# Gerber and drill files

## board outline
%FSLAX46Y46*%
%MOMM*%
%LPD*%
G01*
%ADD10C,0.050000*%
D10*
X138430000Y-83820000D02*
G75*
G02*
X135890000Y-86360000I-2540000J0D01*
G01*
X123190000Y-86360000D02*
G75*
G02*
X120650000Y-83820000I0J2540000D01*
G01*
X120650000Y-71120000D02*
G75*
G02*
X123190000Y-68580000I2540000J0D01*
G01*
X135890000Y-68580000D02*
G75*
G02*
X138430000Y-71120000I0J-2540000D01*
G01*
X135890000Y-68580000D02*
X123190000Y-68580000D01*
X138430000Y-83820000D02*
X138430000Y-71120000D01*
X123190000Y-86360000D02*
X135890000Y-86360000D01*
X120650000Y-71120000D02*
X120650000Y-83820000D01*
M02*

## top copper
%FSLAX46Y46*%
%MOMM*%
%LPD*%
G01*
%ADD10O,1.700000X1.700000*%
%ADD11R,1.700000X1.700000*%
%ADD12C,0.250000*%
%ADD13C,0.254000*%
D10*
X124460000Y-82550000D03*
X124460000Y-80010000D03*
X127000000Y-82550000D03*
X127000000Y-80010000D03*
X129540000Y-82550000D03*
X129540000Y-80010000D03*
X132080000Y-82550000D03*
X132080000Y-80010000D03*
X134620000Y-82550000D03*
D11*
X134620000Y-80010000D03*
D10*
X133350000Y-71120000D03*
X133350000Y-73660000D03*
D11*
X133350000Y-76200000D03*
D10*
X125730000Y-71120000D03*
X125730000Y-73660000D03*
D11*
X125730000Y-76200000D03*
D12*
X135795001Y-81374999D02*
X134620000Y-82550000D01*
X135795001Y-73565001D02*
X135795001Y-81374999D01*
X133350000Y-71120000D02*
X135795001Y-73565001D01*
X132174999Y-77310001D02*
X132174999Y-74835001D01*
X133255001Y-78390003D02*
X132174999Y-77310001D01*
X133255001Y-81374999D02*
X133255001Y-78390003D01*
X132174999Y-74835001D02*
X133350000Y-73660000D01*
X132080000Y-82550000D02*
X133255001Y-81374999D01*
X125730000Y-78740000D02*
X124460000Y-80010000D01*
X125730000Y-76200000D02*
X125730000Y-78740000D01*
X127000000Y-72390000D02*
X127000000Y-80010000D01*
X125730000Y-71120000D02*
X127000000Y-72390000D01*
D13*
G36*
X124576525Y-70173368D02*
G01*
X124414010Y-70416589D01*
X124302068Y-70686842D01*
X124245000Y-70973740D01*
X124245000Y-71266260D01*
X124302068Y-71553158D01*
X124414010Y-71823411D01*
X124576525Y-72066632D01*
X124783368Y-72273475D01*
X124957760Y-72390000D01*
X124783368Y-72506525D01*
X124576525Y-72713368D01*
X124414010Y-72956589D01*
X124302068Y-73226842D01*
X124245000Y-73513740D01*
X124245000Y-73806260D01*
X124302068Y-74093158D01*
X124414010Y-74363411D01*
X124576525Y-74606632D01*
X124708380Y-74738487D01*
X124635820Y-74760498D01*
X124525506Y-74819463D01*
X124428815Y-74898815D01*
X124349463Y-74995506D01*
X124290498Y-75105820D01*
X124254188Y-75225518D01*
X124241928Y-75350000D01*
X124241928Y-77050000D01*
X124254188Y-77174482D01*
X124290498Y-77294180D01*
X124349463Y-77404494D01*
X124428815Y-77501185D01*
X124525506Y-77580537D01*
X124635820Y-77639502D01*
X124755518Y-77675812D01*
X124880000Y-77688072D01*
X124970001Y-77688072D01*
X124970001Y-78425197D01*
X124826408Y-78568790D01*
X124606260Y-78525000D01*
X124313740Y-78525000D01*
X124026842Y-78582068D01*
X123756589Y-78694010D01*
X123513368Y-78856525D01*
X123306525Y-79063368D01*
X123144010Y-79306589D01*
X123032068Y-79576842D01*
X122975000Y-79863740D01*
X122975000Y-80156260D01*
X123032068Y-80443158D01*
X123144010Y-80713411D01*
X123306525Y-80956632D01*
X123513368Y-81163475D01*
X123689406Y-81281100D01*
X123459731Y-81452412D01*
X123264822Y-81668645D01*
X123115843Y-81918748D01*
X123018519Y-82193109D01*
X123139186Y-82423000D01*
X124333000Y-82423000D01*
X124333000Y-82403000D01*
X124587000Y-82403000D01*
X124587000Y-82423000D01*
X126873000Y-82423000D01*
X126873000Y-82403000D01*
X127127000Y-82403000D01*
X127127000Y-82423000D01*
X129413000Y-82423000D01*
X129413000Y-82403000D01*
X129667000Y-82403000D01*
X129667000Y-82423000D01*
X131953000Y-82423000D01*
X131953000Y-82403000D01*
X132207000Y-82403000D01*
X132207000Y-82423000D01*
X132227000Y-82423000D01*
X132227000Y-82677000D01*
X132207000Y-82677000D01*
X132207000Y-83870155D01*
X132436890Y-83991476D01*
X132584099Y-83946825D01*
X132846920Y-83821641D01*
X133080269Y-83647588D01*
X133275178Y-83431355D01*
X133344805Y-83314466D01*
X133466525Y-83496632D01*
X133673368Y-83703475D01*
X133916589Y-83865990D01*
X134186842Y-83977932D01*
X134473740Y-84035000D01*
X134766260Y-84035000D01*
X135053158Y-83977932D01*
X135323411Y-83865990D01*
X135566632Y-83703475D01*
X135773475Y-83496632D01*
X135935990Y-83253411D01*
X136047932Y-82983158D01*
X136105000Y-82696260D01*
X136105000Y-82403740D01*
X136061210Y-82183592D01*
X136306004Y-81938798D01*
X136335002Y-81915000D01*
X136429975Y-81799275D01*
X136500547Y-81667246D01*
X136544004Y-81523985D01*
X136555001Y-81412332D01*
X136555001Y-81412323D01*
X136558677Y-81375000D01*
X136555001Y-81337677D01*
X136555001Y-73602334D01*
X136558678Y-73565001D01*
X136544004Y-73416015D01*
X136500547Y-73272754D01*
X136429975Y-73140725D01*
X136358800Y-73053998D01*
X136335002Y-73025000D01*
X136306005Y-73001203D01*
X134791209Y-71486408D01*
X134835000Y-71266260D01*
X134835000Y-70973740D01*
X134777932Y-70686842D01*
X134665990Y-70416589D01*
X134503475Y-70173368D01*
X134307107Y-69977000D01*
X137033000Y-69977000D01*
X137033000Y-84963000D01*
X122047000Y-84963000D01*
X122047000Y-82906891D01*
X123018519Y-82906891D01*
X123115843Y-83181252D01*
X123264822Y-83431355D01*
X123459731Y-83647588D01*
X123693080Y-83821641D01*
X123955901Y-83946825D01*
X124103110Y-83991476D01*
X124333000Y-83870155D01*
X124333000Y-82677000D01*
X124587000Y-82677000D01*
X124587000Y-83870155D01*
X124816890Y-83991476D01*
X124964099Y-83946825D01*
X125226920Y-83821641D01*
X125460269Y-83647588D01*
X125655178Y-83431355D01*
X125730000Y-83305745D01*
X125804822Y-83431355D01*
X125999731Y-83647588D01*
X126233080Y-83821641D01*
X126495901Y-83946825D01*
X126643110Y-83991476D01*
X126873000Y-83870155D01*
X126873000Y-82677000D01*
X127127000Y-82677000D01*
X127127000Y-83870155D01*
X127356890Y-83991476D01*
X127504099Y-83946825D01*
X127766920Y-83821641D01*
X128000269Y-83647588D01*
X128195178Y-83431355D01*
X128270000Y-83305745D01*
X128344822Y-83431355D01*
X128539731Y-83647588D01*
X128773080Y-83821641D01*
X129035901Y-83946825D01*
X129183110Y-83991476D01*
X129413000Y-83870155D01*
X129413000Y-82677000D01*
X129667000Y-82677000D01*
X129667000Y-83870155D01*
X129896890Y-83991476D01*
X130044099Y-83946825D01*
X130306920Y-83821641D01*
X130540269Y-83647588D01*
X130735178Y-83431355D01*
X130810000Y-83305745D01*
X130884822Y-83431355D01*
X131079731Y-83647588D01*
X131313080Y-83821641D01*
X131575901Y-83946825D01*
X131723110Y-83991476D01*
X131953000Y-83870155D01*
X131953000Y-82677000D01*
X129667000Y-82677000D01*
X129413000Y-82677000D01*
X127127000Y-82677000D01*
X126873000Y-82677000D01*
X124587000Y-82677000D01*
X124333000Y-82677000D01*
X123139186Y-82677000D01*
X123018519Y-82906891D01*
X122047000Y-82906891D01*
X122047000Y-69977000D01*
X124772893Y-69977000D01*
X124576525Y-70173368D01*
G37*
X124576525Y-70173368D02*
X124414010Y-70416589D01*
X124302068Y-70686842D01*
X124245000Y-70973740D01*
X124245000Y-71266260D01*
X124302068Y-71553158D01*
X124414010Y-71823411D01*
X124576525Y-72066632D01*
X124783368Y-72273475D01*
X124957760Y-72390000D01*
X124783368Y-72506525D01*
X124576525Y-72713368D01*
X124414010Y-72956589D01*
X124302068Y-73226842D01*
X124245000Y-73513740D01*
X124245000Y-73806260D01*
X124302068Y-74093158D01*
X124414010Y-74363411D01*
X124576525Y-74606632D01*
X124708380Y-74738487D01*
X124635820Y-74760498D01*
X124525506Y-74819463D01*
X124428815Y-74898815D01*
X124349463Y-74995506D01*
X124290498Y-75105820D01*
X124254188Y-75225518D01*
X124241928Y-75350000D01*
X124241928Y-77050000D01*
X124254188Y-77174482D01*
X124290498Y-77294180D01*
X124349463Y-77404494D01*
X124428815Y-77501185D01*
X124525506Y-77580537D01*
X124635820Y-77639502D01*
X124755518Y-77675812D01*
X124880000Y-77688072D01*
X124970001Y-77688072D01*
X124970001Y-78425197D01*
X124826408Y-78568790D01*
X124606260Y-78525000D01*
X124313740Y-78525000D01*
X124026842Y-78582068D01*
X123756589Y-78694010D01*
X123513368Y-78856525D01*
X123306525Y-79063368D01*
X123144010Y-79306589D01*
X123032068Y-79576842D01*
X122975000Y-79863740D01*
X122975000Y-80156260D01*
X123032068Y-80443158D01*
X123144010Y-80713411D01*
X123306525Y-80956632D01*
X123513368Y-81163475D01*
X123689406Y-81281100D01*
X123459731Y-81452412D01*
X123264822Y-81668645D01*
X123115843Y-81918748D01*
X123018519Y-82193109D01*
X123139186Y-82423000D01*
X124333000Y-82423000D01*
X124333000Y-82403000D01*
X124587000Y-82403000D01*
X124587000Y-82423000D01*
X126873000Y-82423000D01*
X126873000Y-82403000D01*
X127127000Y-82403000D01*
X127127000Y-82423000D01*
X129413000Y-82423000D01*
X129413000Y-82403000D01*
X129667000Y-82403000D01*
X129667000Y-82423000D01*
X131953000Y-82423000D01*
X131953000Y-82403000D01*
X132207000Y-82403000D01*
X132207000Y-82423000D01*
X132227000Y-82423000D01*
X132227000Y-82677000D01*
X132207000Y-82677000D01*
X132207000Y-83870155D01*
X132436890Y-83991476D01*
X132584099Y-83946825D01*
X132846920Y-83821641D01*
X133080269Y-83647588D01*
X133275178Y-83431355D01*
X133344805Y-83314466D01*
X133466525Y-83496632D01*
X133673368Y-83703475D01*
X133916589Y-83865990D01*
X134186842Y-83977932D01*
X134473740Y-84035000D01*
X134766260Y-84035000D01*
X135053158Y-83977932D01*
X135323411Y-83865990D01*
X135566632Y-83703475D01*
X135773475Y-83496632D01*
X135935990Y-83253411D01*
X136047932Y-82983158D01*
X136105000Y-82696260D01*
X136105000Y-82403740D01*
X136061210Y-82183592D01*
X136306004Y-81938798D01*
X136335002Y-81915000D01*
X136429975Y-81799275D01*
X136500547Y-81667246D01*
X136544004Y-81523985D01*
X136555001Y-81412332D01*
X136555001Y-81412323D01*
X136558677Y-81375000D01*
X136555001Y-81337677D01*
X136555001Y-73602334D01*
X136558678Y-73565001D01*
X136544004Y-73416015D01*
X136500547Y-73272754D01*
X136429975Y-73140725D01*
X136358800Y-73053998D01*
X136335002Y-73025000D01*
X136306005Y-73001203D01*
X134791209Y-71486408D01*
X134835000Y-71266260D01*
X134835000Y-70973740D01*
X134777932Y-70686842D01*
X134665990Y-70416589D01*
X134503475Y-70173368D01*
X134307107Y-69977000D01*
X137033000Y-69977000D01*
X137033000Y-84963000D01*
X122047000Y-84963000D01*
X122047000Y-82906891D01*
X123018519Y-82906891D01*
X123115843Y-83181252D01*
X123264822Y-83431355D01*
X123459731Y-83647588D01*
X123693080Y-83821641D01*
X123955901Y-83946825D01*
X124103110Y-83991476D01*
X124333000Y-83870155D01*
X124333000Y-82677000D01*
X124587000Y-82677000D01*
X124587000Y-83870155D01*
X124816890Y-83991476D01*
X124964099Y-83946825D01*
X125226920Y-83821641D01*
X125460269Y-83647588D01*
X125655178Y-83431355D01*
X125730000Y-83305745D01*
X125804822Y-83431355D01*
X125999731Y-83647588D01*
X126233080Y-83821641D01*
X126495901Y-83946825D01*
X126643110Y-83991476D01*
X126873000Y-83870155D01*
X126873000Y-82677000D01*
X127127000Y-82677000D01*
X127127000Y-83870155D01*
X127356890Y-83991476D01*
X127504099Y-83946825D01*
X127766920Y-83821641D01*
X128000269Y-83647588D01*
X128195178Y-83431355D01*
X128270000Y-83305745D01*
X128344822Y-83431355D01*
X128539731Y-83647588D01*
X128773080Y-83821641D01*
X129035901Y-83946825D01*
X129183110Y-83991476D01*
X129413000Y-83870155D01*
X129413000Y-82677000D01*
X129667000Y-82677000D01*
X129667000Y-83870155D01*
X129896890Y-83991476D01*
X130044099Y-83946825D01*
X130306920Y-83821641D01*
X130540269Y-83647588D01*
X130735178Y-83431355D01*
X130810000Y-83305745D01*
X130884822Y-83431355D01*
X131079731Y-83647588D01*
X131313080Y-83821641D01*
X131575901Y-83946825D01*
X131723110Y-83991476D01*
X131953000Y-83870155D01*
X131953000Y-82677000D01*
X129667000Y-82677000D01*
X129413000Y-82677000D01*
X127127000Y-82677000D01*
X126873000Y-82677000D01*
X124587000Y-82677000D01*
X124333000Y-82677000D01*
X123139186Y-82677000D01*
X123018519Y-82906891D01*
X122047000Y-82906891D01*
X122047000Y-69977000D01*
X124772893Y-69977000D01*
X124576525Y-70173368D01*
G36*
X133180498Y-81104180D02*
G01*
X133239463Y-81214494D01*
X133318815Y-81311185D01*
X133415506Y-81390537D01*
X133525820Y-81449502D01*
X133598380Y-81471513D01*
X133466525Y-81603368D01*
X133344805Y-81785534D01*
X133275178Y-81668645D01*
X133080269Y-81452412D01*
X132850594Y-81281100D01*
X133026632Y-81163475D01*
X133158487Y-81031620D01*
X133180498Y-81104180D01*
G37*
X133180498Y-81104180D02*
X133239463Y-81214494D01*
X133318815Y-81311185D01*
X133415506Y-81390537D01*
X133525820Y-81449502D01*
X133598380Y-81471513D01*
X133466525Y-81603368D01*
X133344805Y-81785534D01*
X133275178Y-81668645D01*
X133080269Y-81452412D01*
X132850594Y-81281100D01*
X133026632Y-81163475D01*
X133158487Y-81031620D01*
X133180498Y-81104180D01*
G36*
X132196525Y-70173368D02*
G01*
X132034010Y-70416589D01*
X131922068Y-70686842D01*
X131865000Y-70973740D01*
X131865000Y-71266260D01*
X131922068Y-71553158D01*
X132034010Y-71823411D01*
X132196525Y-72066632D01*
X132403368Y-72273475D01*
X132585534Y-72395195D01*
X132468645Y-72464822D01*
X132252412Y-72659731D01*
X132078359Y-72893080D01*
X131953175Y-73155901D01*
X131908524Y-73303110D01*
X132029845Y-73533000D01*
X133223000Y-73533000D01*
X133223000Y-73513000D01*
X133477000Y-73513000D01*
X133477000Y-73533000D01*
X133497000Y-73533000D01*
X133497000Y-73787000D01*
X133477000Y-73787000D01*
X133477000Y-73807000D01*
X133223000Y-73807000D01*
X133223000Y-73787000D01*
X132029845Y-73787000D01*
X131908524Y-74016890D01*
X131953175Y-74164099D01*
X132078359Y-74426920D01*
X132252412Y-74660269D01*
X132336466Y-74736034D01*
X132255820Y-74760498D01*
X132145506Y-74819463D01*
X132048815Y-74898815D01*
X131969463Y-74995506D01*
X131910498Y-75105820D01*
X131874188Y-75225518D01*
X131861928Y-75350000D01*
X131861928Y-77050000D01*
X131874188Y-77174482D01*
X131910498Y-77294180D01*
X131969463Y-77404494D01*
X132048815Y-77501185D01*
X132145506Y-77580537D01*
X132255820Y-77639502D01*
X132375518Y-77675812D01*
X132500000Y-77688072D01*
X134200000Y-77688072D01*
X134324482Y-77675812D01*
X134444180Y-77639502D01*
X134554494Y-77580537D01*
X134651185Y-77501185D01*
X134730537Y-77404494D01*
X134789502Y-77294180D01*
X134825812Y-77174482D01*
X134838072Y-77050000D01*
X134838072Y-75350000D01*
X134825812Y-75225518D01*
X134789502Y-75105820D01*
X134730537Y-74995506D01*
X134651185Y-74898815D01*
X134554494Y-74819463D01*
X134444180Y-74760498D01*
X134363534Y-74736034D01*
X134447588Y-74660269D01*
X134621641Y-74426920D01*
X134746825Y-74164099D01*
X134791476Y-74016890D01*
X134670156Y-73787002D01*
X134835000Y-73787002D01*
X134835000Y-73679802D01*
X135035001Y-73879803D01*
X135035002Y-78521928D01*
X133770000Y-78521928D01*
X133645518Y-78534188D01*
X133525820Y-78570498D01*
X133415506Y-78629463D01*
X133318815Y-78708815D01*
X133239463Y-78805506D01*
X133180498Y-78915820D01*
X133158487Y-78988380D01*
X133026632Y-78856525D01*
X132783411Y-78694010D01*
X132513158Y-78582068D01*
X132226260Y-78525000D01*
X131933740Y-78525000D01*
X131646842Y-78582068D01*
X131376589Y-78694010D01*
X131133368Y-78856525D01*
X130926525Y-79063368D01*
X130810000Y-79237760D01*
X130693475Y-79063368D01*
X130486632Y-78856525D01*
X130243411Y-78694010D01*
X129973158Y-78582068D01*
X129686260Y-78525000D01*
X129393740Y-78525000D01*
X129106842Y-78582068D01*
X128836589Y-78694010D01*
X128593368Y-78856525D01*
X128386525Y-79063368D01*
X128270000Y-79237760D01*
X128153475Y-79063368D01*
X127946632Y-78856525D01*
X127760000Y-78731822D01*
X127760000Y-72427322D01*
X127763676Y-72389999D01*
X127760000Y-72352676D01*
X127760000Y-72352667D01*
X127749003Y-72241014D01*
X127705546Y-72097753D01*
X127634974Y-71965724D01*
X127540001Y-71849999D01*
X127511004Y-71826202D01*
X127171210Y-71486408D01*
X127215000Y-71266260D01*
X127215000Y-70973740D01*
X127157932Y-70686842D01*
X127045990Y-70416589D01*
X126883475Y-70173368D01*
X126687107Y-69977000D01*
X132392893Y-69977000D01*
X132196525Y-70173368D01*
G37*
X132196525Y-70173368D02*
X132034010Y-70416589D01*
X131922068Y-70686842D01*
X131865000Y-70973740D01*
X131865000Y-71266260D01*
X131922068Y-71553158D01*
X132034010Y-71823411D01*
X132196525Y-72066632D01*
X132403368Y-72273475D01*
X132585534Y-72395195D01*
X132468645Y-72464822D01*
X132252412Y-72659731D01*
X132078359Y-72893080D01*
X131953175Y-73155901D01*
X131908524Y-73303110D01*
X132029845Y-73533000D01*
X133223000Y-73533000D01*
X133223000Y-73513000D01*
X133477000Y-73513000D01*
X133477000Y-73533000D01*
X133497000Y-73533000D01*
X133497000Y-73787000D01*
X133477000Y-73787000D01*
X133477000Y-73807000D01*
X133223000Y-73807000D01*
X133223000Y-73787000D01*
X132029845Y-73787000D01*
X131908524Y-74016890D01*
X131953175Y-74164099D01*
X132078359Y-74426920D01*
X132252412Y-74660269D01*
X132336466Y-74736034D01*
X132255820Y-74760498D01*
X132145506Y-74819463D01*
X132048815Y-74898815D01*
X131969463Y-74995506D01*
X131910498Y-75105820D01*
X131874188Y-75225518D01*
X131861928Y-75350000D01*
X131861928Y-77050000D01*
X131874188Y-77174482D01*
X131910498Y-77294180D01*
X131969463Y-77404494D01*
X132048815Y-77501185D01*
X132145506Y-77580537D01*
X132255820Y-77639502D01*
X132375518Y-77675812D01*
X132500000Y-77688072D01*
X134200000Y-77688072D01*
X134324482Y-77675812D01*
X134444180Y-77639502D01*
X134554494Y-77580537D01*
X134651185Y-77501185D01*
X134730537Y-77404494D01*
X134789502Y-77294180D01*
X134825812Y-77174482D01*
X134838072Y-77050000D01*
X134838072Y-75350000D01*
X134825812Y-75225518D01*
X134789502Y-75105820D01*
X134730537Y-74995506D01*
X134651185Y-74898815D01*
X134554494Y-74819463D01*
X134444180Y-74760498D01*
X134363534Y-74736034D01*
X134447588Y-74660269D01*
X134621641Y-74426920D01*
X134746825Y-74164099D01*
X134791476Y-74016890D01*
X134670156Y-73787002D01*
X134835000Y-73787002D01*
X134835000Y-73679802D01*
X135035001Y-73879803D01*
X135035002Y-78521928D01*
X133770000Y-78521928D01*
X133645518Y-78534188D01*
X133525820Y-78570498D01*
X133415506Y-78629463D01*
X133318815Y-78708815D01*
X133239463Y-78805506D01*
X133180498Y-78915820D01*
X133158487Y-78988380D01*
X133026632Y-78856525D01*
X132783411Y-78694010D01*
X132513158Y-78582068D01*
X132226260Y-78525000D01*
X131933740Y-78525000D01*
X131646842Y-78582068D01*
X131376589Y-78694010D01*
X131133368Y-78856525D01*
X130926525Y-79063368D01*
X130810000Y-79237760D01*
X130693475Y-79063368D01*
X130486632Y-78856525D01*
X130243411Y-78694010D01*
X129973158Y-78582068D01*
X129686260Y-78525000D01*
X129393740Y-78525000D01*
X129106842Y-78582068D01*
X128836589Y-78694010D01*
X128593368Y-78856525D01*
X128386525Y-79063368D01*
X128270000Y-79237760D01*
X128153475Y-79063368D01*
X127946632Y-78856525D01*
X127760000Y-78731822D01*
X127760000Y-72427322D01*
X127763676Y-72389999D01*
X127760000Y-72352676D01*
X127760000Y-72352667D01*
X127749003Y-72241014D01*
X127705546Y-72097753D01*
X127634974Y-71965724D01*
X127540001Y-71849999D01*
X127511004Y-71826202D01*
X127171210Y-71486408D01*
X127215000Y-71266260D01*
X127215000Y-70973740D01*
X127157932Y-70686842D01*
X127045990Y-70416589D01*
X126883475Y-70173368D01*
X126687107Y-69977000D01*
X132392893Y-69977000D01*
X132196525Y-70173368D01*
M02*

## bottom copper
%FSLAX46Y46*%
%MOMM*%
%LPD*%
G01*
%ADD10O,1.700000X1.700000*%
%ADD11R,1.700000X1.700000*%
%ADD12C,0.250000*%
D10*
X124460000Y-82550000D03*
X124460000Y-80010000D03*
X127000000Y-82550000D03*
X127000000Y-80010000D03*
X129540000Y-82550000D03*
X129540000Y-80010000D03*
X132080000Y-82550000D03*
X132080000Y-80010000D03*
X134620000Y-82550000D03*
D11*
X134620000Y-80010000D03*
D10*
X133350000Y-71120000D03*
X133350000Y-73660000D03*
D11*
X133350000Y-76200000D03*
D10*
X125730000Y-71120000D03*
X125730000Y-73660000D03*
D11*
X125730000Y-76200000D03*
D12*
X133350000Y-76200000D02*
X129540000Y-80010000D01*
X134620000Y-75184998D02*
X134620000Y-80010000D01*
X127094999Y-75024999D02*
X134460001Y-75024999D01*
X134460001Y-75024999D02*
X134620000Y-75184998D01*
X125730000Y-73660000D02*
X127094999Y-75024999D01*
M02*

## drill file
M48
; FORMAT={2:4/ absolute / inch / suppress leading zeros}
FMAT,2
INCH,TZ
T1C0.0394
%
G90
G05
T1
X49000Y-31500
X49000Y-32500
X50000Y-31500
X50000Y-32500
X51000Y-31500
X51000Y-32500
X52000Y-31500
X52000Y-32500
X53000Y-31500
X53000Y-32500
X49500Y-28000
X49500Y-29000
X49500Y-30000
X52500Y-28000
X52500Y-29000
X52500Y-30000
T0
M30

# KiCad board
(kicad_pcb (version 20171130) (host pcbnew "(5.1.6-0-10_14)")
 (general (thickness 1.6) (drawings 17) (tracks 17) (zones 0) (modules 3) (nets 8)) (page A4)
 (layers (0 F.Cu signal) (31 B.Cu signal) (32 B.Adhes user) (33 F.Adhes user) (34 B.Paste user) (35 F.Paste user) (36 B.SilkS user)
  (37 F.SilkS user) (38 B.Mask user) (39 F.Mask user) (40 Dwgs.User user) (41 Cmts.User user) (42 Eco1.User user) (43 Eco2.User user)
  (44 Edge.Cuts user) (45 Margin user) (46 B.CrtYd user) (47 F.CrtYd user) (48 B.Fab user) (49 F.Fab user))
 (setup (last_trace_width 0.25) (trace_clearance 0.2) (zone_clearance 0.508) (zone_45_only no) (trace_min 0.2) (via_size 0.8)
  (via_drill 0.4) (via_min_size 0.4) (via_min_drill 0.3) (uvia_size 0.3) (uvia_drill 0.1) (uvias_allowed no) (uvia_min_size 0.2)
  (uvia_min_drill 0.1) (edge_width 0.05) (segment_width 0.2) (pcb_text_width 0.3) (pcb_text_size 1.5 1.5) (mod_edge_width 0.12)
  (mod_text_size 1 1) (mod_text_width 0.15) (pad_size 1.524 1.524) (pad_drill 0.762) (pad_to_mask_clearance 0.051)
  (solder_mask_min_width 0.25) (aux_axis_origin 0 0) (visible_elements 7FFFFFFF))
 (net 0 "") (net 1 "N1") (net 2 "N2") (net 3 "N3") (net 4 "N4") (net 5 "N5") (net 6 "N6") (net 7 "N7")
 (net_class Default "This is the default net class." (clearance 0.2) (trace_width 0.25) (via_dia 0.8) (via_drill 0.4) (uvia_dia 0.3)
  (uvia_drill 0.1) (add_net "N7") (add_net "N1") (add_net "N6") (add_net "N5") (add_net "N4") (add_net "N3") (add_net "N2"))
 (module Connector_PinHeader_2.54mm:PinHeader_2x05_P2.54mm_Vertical (layer F.Cu) (at 134.62 80.01 270)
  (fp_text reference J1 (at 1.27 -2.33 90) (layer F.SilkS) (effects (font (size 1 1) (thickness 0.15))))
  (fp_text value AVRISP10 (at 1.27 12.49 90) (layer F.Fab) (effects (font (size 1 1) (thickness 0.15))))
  (pad 10 thru_hole oval (at 2.54 10.16 270) (size 1.7 1.7) (drill 1) (layers *.Cu *.Mask) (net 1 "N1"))
  (pad 9 thru_hole oval (at 0 10.16 270) (size 1.7 1.7) (drill 1) (layers *.Cu *.Mask) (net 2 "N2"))
  (pad 8 thru_hole oval (at 2.54 7.62 270) (size 1.7 1.7) (drill 1) (layers *.Cu *.Mask) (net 1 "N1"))
  (pad 7 thru_hole oval (at 0 7.62 270) (size 1.7 1.7) (drill 1) (layers *.Cu *.Mask) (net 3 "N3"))
  (pad 6 thru_hole oval (at 2.54 5.08 270) (size 1.7 1.7) (drill 1) (layers *.Cu *.Mask) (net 1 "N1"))
  (pad 5 thru_hole oval (at 0 5.08 270) (size 1.7 1.7) (drill 1) (layers *.Cu *.Mask) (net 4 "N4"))
  (pad 4 thru_hole oval (at 2.54 2.54 270) (size 1.7 1.7) (drill 1) (layers *.Cu *.Mask) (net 1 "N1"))
  (pad 3 thru_hole oval (at 0 2.54 270) (size 1.7 1.7) (drill 1) (layers *.Cu *.Mask) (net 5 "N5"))
  (pad 2 thru_hole oval (at 2.54 0 270) (size 1.7 1.7) (drill 1) (layers *.Cu *.Mask) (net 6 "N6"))
  (pad 1 thru_hole rect (at 0 0 270) (size 1.7 1.7) (drill 1) (layers *.Cu *.Mask) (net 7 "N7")))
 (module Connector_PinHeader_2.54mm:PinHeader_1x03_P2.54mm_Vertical (layer B.Cu) (at 133.35 76.2)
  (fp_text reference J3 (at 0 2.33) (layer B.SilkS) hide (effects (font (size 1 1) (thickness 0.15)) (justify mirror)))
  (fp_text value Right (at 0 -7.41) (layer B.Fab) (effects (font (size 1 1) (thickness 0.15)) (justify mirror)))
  (pad 3 thru_hole oval (at 0 -5.08) (size 1.7 1.7) (drill 1) (layers *.Cu *.Mask) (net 6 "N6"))
  (pad 2 thru_hole oval (at 0 -2.54) (size 1.7 1.7) (drill 1) (layers *.Cu *.Mask) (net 1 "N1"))
  (pad 1 thru_hole rect (at 0 0) (size 1.7 1.7) (drill 1) (layers *.Cu *.Mask) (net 4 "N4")))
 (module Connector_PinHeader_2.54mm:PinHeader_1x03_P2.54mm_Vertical (layer B.Cu) (at 125.73 76.2)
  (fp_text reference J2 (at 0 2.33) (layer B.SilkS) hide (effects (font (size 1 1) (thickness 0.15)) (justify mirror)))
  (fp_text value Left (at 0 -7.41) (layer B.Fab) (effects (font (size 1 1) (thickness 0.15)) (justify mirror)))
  (pad 3 thru_hole oval (at 0 -5.08) (size 1.7 1.7) (drill 1) (layers *.Cu *.Mask) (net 3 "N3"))
  (pad 2 thru_hole oval (at 0 -2.54) (size 1.7 1.7) (drill 1) (layers *.Cu *.Mask) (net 7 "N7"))
  (pad 1 thru_hole rect (at 0 0) (size 1.7 1.7) (drill 1) (layers *.Cu *.Mask) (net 2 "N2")))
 (gr_arc (start 135.89 83.82) (end 135.89 86.36) (angle -90) (layer Edge.Cuts) (width 0.05))
 (gr_arc (start 123.19 83.82) (end 120.65 83.82) (angle -90) (layer Edge.Cuts) (width 0.05))
 (gr_arc (start 123.19 71.12) (end 123.19 68.58) (angle -90) (layer Edge.Cuts) (width 0.05))
 (gr_arc (start 135.89 71.12) (end 138.43 71.12) (angle -90) (layer Edge.Cuts) (width 0.05))
 (gr_line (start 135.89 68.58) (end 123.19 68.58) (layer Edge.Cuts) (width 0.05))
 (gr_line (start 138.43 83.82) (end 138.43 71.12) (layer Edge.Cuts) (width 0.05))
 (gr_line (start 123.19 86.36) (end 135.89 86.36) (layer Edge.Cuts) (width 0.05))
 (gr_line (start 120.65 71.12) (end 120.65 83.82) (layer Edge.Cuts) (width 0.05))
 (segment (start 133.35 76.2) (end 129.54 80.01) (width 0.25) (layer B.Cu) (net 4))
 (segment (start 135.795001 81.374999) (end 134.62 82.55) (width 0.25) (layer F.Cu) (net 6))
 (segment (start 135.795001 73.565001) (end 135.795001 81.374999) (width 0.25) (layer F.Cu) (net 6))
 (segment (start 133.35 71.12) (end 135.795001 73.565001) (width 0.25) (layer F.Cu) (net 6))
 (segment (start 134.62 75.184998) (end 134.62 80.01) (width 0.25) (layer B.Cu) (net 7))
 (segment (start 127.094999 75.024999) (end 134.460001 75.024999) (width 0.25) (layer B.Cu) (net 7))
 (segment (start 134.460001 75.024999) (end 134.62 75.184998) (width 0.25) (layer B.Cu) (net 7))
 (segment (start 125.73 73.66) (end 127.094999 75.024999) (width 0.25) (layer B.Cu) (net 7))
 (segment (start 132.174999 77.310001) (end 132.174999 74.835001) (width 0.25) (layer F.Cu) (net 1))
 (segment (start 133.255001 78.390003) (end 132.174999 77.310001) (width 0.25) (layer F.Cu) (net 1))
 (segment (start 133.255001 81.374999) (end 133.255001 78.390003) (width 0.25) (layer F.Cu) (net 1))
 (segment (start 132.174999 74.835001) (end 133.35 73.66) (width 0.25) (layer F.Cu) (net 1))
 (segment (start 132.08 82.55) (end 133.255001 81.374999) (width 0.25) (layer F.Cu) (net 1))
 (segment (start 125.73 78.74) (end 124.46 80.01) (width 0.25) (layer F.Cu) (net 2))
 (segment (start 125.73 76.2) (end 125.73 78.74) (width 0.25) (layer F.Cu) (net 2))
 (segment (start 127 72.39) (end 127 80.01) (width 0.25) (layer F.Cu) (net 3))
 (segment (start 125.73 71.12) (end 127 72.39) (width 0.25) (layer F.Cu) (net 3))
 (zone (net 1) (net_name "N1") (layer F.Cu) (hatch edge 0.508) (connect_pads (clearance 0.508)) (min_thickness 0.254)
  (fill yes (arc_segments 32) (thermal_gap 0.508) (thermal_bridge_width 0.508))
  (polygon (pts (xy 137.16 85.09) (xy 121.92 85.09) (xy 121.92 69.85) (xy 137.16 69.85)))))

